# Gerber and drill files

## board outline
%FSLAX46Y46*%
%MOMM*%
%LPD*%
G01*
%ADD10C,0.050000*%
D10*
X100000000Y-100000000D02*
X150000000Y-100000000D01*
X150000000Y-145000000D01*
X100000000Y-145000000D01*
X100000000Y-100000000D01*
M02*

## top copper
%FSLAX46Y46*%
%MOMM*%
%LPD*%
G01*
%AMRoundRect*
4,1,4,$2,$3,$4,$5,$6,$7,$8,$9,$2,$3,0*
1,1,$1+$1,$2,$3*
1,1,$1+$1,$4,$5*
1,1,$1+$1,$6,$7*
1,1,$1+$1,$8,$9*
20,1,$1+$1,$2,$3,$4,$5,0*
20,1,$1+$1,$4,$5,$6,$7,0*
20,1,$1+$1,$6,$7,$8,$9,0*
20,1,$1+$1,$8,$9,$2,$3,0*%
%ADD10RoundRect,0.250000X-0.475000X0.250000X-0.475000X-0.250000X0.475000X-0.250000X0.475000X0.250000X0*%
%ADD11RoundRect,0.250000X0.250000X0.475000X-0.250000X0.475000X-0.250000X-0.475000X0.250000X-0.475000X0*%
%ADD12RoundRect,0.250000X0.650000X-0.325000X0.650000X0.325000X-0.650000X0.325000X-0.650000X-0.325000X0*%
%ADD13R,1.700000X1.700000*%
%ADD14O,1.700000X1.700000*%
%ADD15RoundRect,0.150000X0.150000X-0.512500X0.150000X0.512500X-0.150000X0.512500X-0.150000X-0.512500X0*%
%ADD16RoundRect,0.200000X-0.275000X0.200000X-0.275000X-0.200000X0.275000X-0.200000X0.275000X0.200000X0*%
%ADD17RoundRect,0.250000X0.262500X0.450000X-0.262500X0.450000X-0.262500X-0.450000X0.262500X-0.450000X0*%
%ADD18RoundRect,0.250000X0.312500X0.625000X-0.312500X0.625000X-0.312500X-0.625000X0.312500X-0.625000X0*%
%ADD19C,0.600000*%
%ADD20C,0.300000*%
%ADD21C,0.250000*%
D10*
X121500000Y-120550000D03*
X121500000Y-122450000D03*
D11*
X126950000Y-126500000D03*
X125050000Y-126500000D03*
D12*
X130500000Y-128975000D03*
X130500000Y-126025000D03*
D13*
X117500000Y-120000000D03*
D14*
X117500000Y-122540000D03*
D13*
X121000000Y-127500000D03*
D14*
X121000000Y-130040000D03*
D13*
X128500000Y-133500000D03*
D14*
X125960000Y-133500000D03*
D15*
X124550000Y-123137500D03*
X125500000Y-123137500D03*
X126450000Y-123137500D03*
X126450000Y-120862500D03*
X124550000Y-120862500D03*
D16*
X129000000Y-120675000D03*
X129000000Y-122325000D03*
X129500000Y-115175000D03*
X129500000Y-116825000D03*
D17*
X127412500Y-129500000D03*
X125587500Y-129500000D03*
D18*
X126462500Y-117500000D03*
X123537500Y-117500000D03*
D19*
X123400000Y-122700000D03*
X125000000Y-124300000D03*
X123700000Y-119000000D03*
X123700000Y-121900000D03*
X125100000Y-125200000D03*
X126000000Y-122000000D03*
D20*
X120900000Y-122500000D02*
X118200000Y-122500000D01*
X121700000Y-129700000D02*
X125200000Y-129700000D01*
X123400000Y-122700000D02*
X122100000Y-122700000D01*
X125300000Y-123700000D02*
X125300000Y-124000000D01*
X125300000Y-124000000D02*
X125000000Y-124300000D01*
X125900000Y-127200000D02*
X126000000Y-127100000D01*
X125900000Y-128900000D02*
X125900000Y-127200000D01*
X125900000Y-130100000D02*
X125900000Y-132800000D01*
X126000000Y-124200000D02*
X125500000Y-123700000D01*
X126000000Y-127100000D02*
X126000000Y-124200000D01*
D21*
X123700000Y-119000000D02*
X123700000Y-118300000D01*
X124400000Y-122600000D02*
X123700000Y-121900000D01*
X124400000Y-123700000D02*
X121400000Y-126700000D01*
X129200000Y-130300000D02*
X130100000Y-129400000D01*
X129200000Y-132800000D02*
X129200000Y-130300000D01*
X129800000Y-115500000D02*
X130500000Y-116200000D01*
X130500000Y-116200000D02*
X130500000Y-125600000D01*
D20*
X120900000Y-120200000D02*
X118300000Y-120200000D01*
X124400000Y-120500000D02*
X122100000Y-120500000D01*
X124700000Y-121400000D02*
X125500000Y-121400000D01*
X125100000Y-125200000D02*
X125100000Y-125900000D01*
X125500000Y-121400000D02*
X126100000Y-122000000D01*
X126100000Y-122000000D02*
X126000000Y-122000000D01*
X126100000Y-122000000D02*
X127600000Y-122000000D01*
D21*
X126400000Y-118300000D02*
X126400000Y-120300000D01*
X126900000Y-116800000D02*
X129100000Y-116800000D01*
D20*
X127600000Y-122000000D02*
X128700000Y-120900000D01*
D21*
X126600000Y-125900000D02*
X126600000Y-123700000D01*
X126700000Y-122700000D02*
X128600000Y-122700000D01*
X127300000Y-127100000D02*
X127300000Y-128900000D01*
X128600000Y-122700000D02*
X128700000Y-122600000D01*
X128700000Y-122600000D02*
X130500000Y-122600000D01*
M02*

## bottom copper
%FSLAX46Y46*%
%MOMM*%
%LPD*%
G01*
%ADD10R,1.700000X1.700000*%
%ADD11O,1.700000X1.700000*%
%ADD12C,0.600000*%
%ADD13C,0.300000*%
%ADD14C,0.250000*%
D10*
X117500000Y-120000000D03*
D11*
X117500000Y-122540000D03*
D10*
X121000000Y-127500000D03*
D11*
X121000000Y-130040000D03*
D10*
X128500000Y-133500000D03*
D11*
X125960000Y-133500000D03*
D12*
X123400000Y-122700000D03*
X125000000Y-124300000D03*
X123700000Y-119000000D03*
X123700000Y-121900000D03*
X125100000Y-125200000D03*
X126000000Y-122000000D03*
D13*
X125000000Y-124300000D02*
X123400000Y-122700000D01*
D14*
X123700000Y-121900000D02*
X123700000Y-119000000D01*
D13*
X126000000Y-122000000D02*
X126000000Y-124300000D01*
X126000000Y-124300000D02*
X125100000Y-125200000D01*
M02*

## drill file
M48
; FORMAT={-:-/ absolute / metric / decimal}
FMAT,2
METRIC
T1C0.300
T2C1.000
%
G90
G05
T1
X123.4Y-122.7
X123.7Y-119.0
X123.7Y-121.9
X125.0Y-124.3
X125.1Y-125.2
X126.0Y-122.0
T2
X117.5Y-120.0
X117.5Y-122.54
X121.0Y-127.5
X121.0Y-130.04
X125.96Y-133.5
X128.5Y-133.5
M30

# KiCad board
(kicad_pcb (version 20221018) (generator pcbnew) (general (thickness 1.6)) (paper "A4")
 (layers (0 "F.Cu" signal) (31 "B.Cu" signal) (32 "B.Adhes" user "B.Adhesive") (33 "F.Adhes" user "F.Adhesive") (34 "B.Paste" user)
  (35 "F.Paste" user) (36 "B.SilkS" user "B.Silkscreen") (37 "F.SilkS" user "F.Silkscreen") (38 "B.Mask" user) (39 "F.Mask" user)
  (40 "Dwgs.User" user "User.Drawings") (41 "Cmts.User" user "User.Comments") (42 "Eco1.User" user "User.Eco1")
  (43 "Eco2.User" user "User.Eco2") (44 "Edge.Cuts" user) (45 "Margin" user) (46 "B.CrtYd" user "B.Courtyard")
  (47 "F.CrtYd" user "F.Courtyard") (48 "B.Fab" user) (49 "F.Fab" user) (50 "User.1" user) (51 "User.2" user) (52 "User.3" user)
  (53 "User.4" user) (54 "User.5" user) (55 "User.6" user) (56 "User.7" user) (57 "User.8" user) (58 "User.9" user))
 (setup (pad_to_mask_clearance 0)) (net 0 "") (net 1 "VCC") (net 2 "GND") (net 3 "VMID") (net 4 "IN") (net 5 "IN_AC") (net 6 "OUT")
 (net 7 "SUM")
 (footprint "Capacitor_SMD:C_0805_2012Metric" (layer "F.Cu") (at 121.5 121.5 -90)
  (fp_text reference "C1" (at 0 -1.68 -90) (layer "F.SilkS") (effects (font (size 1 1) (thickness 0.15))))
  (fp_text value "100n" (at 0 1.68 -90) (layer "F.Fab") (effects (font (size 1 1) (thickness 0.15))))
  (pad "1" smd roundrect (at -0.95 0 270) (size 1 1.45) (layers "F.Cu" "F.Paste" "F.Mask") (roundrect_rratio 0.25) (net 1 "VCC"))
  (pad "2" smd roundrect (at 0.95 0 270) (size 1 1.45) (layers "F.Cu" "F.Paste" "F.Mask") (roundrect_rratio 0.25) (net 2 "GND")))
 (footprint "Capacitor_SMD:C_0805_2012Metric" (layer "F.Cu") (at 126 126.5 180)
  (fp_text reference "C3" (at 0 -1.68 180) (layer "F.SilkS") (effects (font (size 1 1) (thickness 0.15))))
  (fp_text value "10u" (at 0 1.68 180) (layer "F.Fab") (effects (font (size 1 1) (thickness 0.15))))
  (pad "1" smd roundrect (at -0.95 0 180) (size 1 1.45) (layers "F.Cu" "F.Paste" "F.Mask") (roundrect_rratio 0.25) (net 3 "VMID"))
  (pad "2" smd roundrect (at 0.95 0 180) (size 1 1.45) (layers "F.Cu" "F.Paste" "F.Mask") (roundrect_rratio 0.25) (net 1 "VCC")))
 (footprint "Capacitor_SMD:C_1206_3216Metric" (layer "F.Cu") (at 130.5 127.5 90)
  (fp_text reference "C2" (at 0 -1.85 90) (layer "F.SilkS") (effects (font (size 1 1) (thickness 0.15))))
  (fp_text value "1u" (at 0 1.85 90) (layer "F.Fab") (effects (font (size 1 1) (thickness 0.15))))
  (pad "1" smd roundrect (at -1.475 0 90) (size 1.15 1.8) (layers "F.Cu" "F.Paste" "F.Mask") (roundrect_rratio 0.217391) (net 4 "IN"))
  (pad "2" smd roundrect (at 1.475 0 90) (size 1.15 1.8) (layers "F.Cu" "F.Paste" "F.Mask") (roundrect_rratio 0.217391) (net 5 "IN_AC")))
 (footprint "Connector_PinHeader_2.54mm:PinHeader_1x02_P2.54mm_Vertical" (layer "F.Cu") (at 117.5 120)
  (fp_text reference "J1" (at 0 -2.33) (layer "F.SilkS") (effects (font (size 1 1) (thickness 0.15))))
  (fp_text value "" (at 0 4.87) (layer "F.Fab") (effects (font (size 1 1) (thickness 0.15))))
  (pad "1" thru_hole rect (at 0 0) (size 1.7 1.7) (drill 1) (layers "*.Cu" "*.Mask") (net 1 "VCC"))
  (pad "2" thru_hole oval (at 0 2.54) (size 1.7 1.7) (drill 1) (layers "*.Cu" "*.Mask") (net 2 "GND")))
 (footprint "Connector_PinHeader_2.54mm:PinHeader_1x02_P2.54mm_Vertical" (layer "F.Cu") (at 121 127.5)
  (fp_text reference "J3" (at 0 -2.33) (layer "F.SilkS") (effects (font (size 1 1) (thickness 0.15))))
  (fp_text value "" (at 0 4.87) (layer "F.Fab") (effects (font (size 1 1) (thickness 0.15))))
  (pad "1" thru_hole rect (at 0 0) (size 1.7 1.7) (drill 1) (layers "*.Cu" "*.Mask") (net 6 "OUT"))
  (pad "2" thru_hole oval (at 0 2.54) (size 1.7 1.7) (drill 1) (layers "*.Cu" "*.Mask") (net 2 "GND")))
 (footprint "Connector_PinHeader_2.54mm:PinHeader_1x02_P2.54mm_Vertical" (layer "F.Cu") (at 128.5 133.5 -90)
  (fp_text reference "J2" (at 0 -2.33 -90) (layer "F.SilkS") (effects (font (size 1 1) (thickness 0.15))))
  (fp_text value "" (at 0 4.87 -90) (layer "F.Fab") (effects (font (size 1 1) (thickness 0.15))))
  (pad "1" thru_hole rect (at 0 0 270) (size 1.7 1.7) (drill 1) (layers "*.Cu" "*.Mask") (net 4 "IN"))
  (pad "2" thru_hole oval (at 0 2.54 270) (size 1.7 1.7) (drill 1) (layers "*.Cu" "*.Mask") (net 2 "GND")))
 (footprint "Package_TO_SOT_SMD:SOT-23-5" (layer "F.Cu") (at 125.5 122 90)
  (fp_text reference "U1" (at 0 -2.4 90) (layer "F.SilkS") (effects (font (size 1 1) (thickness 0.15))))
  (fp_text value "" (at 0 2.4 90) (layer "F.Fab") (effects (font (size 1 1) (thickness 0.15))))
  (pad "1" smd roundrect (at -1.1375 -0.95 90) (size 1.325 0.6) (layers "F.Cu" "F.Paste" "F.Mask") (roundrect_rratio 0.25) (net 6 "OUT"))
  (pad "2" smd roundrect (at -1.1375 0 90) (size 1.325 0.6) (layers "F.Cu" "F.Paste" "F.Mask") (roundrect_rratio 0.25) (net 2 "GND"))
  (pad "3" smd roundrect (at -1.1375 0.95 90) (size 1.325 0.6) (layers "F.Cu" "F.Paste" "F.Mask") (roundrect_rratio 0.25) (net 3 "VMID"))
  (pad "4" smd roundrect (at 1.1375 0.95 90) (size 1.325 0.6) (layers "F.Cu" "F.Paste" "F.Mask") (roundrect_rratio 0.25) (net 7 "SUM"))
  (pad "5" smd roundrect (at 1.1375 -0.95 90) (size 1.325 0.6) (layers "F.Cu" "F.Paste" "F.Mask") (roundrect_rratio 0.25) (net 1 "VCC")))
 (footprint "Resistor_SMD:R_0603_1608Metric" (layer "F.Cu") (at 129 121.5 -90)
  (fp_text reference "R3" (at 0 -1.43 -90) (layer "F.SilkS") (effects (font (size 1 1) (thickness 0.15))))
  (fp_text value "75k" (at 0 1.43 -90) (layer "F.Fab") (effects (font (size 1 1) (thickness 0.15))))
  (pad "1" smd roundrect (at -0.825 0 270) (size 0.8 0.95) (layers "F.Cu" "F.Paste" "F.Mask") (roundrect_rratio 0.25) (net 1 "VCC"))
  (pad "2" smd roundrect (at 0.825 0 270) (size 0.8 0.95) (layers "F.Cu" "F.Paste" "F.Mask") (roundrect_rratio 0.25) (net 3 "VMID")))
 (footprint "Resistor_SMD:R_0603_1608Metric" (layer "F.Cu") (at 129.5 116 -90)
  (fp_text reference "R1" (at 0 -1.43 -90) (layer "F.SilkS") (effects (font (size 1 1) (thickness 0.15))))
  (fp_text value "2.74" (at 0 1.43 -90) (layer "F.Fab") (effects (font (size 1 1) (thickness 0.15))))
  (pad "1" smd roundrect (at -0.825 0 270) (size 0.8 0.95) (layers "F.Cu" "F.Paste" "F.Mask") (roundrect_rratio 0.25) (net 5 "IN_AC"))
  (pad "2" smd roundrect (at 0.825 0 270) (size 0.8 0.95) (layers "F.Cu" "F.Paste" "F.Mask") (roundrect_rratio 0.25) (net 7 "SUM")))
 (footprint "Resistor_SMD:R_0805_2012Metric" (layer "F.Cu") (at 126.5 129.5 180)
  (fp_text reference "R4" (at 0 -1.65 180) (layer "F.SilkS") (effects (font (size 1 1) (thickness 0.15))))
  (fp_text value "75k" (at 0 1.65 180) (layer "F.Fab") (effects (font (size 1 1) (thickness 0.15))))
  (pad "1" smd roundrect (at -0.9125 0 180) (size 1.025 1.4) (layers "F.Cu" "F.Paste" "F.Mask") (roundrect_rratio 0.243902) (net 3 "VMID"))
  (pad "2" smd roundrect (at 0.9125 0 180) (size 1.025 1.4) (layers "F.Cu" "F.Paste" "F.Mask") (roundrect_rratio 0.243902) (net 2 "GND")))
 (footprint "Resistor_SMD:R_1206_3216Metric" (layer "F.Cu") (at 125 117.5 180)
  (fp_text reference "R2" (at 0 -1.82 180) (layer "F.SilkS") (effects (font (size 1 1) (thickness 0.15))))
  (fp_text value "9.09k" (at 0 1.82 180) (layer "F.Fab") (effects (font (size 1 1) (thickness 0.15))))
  (pad "1" smd roundrect (at -1.4625 0 180) (size 1.125 1.75) (layers "F.Cu" "F.Paste" "F.Mask") (roundrect_rratio 0.222222) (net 7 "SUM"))
  (pad "2" smd roundrect (at 1.4625 0 180) (size 1.125 1.75) (layers "F.Cu" "F.Paste" "F.Mask") (roundrect_rratio 0.222222) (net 6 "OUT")))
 (gr_rect (start 100 100) (end 150 145) (stroke (width 0.05) (type default)) (fill none) (layer "Edge.Cuts"))
 (segment (start 120.9 122.5) (end 118.2 122.5) (width 0.3) (layer "F.Cu") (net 2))
 (segment (start 121.7 129.7) (end 125.2 129.7) (width 0.3) (layer "F.Cu") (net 2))
 (segment (start 123.4 122.7) (end 122.1 122.7) (width 0.3) (layer "F.Cu") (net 2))
 (segment (start 125.3 123.7) (end 125.3 124) (width 0.3) (layer "F.Cu") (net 2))
 (segment (start 125.3 124) (end 125 124.3) (width 0.3) (layer "F.Cu") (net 2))
 (segment (start 125.9 127.2) (end 126 127.1) (width 0.3) (layer "F.Cu") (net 2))
 (segment (start 125.9 128.9) (end 125.9 127.2) (width 0.3) (layer "F.Cu") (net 2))
 (segment (start 125.9 130.1) (end 125.9 132.8) (width 0.3) (layer "F.Cu") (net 2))
 (segment (start 126 124.2) (end 125.5 123.7) (width 0.3) (layer "F.Cu") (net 2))
 (segment (start 126 127.1) (end 126 124.2) (width 0.3) (layer "F.Cu") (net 2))
 (via (at 123.4 122.7) (size 0.6) (drill 0.3) (layers "F.Cu" "B.Cu") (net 2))
 (via (at 125 124.3) (size 0.6) (drill 0.3) (layers "F.Cu" "B.Cu") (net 2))
 (segment (start 123.7 119) (end 123.7 118.3) (width 0.25) (layer "F.Cu") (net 6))
 (segment (start 124.4 122.6) (end 123.7 121.9) (width 0.25) (layer "F.Cu") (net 6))
 (segment (start 124.4 123.7) (end 121.4 126.7) (width 0.25) (layer "F.Cu") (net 6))
 (segment (start 125 124.3) (end 123.4 122.7) (width 0.3) (layer "B.Cu") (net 2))
 (segment (start 129.2 130.3) (end 130.1 129.4) (width 0.25) (layer "F.Cu") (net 4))
 (segment (start 129.2 132.8) (end 129.2 130.3) (width 0.25) (layer "F.Cu") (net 4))
 (segment (start 129.8 115.5) (end 130.5 116.2) (width 0.25) (layer "F.Cu") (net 5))
 (segment (start 130.5 116.2) (end 130.5 125.6) (width 0.25) (layer "F.Cu") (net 5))
 (via (at 123.7 119) (size 0.6) (drill 0.3) (layers "F.Cu" "B.Cu") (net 6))
 (via (at 123.7 121.9) (size 0.6) (drill 0.3) (layers "F.Cu" "B.Cu") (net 6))
 (segment (start 120.9 120.2) (end 118.3 120.2) (width 0.3) (layer "F.Cu") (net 1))
 (segment (start 123.7 121.9) (end 123.7 119) (width 0.25) (layer "B.Cu") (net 6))
 (segment (start 124.4 120.5) (end 122.1 120.5) (width 0.3) (layer "F.Cu") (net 1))
 (segment (start 124.7 121.4) (end 125.5 121.4) (width 0.3) (layer "F.Cu") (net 1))
 (segment (start 125.1 125.2) (end 125.1 125.9) (width 0.3) (layer "F.Cu") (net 1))
 (segment (start 125.5 121.4) (end 126.1 122) (width 0.3) (layer "F.Cu") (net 1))
 (segment (start 126.1 122) (end 126 122) (width 0.3) (layer "F.Cu") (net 1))
 (segment (start 126.1 122) (end 127.6 122) (width 0.3) (layer "F.Cu") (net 1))
 (segment (start 126.4 118.3) (end 126.4 120.3) (width 0.25) (layer "F.Cu") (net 7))
 (segment (start 126.9 116.8) (end 129.1 116.8) (width 0.25) (layer "F.Cu") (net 7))
 (segment (start 127.6 122) (end 128.7 120.9) (width 0.3) (layer "F.Cu") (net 1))
 (via (at 125.1 125.2) (size 0.6) (drill 0.3) (layers "F.Cu" "B.Cu") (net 1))
 (via (at 126 122) (size 0.6) (drill 0.3) (layers "F.Cu" "B.Cu") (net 1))
 (segment (start 126 122) (end 126 124.3) (width 0.3) (layer "B.Cu") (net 1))
 (segment (start 126 124.3) (end 125.1 125.2) (width 0.3) (layer "B.Cu") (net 1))
 (segment (start 126.6 125.9) (end 126.6 123.7) (width 0.25) (layer "F.Cu") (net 3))
 (segment (start 126.7 122.7) (end 128.6 122.7) (width 0.25) (layer "F.Cu") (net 3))
 (segment (start 127.3 127.1) (end 127.3 128.9) (width 0.25) (layer "F.Cu") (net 3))
 (segment (start 128.6 122.7) (end 128.7 122.6) (width 0.25) (layer "F.Cu") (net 3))
 (segment (start 128.7 122.6) (end 130.5 122.6) (width 0.25) (layer "F.Cu") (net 3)))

